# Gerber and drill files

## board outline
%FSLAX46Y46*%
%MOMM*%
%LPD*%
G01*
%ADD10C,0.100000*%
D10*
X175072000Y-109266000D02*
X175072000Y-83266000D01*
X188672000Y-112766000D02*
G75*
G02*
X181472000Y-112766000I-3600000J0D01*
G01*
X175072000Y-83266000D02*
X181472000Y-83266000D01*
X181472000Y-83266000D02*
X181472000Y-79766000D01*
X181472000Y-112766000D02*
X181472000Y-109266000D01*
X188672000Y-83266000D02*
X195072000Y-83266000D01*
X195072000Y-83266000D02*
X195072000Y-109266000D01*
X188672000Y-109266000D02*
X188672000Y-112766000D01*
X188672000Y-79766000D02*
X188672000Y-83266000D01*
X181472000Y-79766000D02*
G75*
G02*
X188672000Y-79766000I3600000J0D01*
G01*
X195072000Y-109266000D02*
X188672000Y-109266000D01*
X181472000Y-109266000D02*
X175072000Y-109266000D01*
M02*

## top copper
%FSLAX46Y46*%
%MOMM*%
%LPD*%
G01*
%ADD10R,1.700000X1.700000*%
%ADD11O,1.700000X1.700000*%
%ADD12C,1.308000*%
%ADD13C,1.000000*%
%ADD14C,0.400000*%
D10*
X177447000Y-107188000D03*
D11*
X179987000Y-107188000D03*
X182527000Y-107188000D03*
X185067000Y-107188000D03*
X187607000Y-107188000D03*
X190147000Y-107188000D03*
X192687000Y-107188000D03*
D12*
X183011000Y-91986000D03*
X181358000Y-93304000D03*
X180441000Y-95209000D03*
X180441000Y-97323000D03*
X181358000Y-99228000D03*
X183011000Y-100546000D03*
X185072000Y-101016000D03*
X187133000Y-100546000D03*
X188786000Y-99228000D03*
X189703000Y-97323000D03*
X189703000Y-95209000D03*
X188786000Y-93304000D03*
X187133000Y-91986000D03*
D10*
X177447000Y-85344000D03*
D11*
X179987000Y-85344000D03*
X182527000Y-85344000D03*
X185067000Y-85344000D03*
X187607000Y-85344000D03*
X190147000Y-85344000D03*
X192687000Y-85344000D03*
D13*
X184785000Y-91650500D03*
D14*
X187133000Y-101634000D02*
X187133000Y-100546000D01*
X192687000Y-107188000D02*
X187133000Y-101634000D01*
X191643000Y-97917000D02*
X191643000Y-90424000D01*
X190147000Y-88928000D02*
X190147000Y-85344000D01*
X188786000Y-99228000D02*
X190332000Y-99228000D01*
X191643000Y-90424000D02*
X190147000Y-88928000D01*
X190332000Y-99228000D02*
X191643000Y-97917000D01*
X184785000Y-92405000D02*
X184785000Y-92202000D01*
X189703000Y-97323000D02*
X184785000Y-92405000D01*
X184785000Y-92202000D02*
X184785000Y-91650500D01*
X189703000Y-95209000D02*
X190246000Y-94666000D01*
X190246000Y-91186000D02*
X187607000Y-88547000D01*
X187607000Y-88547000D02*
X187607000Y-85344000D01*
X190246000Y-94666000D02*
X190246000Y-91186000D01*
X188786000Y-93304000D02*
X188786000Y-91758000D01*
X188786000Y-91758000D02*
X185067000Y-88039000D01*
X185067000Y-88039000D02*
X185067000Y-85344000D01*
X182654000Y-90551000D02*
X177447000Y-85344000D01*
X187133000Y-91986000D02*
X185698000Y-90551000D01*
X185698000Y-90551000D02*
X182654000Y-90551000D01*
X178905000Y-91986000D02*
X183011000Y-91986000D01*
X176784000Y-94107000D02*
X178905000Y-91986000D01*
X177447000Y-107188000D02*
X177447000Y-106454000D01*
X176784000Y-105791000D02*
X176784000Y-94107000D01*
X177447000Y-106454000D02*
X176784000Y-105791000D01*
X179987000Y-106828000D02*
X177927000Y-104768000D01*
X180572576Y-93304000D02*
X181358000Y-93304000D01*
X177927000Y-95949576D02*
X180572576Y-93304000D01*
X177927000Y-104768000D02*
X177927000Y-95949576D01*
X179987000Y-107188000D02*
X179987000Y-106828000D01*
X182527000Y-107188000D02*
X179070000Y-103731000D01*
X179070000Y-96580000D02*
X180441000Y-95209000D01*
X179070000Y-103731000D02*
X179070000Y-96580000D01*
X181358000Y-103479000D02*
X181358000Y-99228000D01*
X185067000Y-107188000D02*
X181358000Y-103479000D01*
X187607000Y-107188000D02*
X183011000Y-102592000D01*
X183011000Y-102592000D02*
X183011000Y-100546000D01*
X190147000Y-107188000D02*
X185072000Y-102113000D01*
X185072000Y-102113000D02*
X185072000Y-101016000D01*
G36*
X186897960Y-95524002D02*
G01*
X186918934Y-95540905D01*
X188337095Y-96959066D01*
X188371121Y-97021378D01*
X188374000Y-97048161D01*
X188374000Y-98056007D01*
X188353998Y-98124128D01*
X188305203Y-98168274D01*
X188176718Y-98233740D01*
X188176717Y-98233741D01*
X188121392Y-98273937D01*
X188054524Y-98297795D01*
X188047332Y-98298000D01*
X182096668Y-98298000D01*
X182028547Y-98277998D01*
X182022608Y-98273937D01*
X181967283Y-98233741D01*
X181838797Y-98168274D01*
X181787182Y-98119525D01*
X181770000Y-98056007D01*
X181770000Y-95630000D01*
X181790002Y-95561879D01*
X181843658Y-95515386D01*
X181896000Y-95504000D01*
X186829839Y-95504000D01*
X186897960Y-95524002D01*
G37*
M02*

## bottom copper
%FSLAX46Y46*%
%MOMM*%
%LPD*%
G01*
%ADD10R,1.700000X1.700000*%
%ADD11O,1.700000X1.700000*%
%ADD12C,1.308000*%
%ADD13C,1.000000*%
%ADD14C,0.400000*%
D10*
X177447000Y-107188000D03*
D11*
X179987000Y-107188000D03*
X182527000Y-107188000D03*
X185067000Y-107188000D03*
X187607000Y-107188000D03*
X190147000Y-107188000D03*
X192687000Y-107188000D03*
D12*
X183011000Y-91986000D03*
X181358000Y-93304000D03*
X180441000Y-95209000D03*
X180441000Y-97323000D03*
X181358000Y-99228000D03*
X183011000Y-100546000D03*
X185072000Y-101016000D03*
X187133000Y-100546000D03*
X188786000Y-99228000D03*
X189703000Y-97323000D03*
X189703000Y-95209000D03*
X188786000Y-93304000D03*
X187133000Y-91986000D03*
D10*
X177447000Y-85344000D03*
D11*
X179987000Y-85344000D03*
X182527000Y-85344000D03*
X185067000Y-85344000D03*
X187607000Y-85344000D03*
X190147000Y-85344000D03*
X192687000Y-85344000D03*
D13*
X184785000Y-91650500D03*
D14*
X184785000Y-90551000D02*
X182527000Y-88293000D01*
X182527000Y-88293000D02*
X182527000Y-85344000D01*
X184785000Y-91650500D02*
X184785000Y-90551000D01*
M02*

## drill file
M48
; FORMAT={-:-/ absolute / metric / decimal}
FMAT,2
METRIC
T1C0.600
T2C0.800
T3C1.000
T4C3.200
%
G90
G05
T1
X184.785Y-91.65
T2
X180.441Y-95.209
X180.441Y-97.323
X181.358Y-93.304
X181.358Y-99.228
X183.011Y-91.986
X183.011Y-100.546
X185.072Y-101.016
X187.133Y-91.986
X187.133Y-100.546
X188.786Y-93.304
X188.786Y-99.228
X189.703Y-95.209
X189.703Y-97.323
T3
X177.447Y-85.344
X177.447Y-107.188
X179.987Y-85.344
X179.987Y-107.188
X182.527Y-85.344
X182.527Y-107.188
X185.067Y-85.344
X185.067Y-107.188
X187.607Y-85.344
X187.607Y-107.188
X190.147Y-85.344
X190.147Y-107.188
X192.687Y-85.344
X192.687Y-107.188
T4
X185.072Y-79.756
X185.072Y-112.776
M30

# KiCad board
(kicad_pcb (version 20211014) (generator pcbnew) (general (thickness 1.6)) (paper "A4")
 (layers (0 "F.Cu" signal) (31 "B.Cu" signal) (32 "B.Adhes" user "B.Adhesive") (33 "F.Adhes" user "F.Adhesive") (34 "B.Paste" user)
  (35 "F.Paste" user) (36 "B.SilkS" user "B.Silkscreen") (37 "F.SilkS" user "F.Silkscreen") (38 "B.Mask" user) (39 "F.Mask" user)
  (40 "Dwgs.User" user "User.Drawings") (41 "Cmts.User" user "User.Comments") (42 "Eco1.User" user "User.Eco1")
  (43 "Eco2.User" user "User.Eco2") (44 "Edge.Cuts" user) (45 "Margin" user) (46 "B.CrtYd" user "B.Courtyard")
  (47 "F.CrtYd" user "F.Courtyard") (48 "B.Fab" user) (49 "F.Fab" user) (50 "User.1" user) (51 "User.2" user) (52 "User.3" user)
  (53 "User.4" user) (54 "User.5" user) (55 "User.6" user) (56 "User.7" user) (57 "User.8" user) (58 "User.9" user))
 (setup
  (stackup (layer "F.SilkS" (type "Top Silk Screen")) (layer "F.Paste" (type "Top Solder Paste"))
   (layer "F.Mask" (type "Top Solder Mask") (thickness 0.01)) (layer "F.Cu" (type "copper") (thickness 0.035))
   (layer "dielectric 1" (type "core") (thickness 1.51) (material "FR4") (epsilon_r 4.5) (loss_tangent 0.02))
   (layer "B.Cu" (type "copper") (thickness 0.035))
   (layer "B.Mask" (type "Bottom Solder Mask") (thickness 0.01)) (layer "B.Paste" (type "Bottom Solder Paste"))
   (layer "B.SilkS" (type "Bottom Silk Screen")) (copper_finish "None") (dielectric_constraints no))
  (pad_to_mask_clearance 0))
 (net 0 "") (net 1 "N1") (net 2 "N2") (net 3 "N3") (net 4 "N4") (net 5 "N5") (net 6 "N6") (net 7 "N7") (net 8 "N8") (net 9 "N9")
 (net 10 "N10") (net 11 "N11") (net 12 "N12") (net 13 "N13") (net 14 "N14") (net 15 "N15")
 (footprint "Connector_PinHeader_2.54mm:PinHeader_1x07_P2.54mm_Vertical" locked (layer "F.Cu") (at 177.447 107.188 90)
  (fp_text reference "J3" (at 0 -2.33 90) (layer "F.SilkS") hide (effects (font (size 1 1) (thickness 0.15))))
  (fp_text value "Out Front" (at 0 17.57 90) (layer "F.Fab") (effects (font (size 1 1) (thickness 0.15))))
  (pad "1" thru_hole rect locked (at 0 0 90) (size 1.7 1.7) (drill 1) (layers *.Cu *.Mask) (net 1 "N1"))
  (pad "2" thru_hole oval locked (at 0 2.54 90) (size 1.7 1.7) (drill 1) (layers *.Cu *.Mask) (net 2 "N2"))
  (pad "3" thru_hole oval locked (at 0 5.08 90) (size 1.7 1.7) (drill 1) (layers *.Cu *.Mask) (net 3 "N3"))
  (pad "4" thru_hole oval locked (at 0 7.62 90) (size 1.7 1.7) (drill 1) (layers *.Cu *.Mask) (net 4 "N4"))
  (pad "5" thru_hole oval locked (at 0 10.16 90) (size 1.7 1.7) (drill 1) (layers *.Cu *.Mask) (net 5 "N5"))
  (pad "6" thru_hole oval locked (at 0 12.7 90) (size 1.7 1.7) (drill 1) (layers *.Cu *.Mask) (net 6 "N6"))
  (pad "7" thru_hole oval locked (at 0 15.24 90) (size 1.7 1.7) (drill 1) (layers *.Cu *.Mask) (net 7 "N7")))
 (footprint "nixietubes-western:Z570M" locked (layer "F.Cu") (at 185.072 96.266 180)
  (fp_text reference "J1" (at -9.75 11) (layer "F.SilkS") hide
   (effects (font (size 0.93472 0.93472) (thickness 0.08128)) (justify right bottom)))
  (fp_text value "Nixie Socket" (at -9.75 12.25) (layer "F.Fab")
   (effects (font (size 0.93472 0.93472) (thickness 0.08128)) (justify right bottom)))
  (pad "1" thru_hole circle locked (at 2.061 4.28 180) (size 1.308 1.308) (drill 0.8) (layers *.Cu *.Mask) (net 1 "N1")
   (solder_mask_margin 0.1016))
  (pad "2" thru_hole circle locked (at 3.714 2.962 180) (size 1.308 1.308) (drill 0.8) (layers *.Cu *.Mask) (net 2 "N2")
   (solder_mask_margin 0.1016))
  (pad "3" thru_hole circle locked (at 4.631 1.057 180) (size 1.308 1.308) (drill 0.8) (layers *.Cu *.Mask) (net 3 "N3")
   (solder_mask_margin 0.1016))
  (pad "4" thru_hole circle locked (at 4.631 -1.057 180) (size 1.308 1.308) (drill 0.8) (layers *.Cu *.Mask) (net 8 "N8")
   (solder_mask_margin 0.1016))
  (pad "5" thru_hole circle locked (at 3.714 -2.962 180) (size 1.308 1.308) (drill 0.8) (layers *.Cu *.Mask) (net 4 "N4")
   (solder_mask_margin 0.1016))
  (pad "6" thru_hole circle locked (at 2.061 -4.28 180) (size 1.308 1.308) (drill 0.8) (layers *.Cu *.Mask) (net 5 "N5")
   (solder_mask_margin 0.1016))
  (pad "7" thru_hole circle locked (at 0 -4.75 180) (size 1.308 1.308) (drill 0.8) (layers *.Cu *.Mask) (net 6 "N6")
   (solder_mask_margin 0.1016))
  (pad "8" thru_hole circle locked (at -2.061 -4.28 180) (size 1.308 1.308) (drill 0.8) (layers *.Cu *.Mask) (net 7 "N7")
   (solder_mask_margin 0.1016))
  (pad "9" thru_hole circle locked (at -3.714 -2.962 180) (size 1.308 1.308) (drill 0.8) (layers *.Cu *.Mask) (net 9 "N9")
   (solder_mask_margin 0.1016))
  (pad "10" thru_hole circle locked (at -4.631 -1.057 180) (size 1.308 1.308) (drill 0.8) (layers *.Cu *.Mask) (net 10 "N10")
   (solder_mask_margin 0.1016))
  (pad "11" thru_hole circle locked (at -4.631 1.057 180) (size 1.308 1.308) (drill 0.8) (layers *.Cu *.Mask) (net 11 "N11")
   (solder_mask_margin 0.1016))
  (pad "12" thru_hole circle locked (at -3.714 2.962 180) (size 1.308 1.308) (drill 0.8) (layers *.Cu *.Mask) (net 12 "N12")
   (solder_mask_margin 0.1016))
  (pad "13" thru_hole circle locked (at -2.061 4.28 180) (size 1.308 1.308) (drill 0.8) (layers *.Cu *.Mask) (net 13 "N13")
   (solder_mask_margin 0.1016)))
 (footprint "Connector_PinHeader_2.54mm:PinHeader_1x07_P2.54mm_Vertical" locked (layer "F.Cu") (at 177.447 85.344 90)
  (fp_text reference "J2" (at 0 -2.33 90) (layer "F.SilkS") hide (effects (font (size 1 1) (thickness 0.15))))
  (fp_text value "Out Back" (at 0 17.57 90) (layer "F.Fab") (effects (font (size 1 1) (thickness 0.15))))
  (pad "1" thru_hole rect locked (at 0 0 90) (size 1.7 1.7) (drill 1) (layers *.Cu *.Mask) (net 13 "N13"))
  (pad "2" thru_hole oval locked (at 0 2.54 90) (size 1.7 1.7) (drill 1) (layers *.Cu *.Mask) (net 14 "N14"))
  (pad "3" thru_hole oval locked (at 0 5.08 90) (size 1.7 1.7) (drill 1) (layers *.Cu *.Mask) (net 10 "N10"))
  (pad "4" thru_hole oval locked (at 0 7.62 90) (size 1.7 1.7) (drill 1) (layers *.Cu *.Mask) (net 12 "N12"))
  (pad "5" thru_hole oval locked (at 0 10.16 90) (size 1.7 1.7) (drill 1) (layers *.Cu *.Mask) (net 11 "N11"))
  (pad "6" thru_hole oval locked (at 0 12.7 90) (size 1.7 1.7) (drill 1) (layers *.Cu *.Mask) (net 9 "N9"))
  (pad "7" thru_hole oval locked (at 0 15.24 90) (size 1.7 1.7) (drill 1) (layers *.Cu *.Mask) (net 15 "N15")))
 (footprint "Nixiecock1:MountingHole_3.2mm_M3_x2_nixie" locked (layer "F.Cu") (at 185.072 96.266 90)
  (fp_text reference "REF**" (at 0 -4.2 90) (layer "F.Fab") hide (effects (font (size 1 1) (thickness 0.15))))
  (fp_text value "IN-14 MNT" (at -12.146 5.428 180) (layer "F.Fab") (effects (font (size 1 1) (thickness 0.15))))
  (pad "" np_thru_hole circle locked (at -16.51 0 90) (size 3.2 3.2) (drill 3.2) (layers F&B.Cu *.Mask))
  (pad "" np_thru_hole circle locked (at 16.51 0 90) (size 3.2 3.2) (drill 3.2) (layers F&B.Cu *.Mask)))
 (gr_line locked (start 175.072 109.266) (end 175.072 83.266) (layer "Edge.Cuts") (width 0.1))
 (gr_arc locked (start 188.672 112.766) (mid 185.072 116.366) (end 181.472 112.766) (layer "Edge.Cuts") (width 0.1))
 (gr_line locked (start 175.072 83.266) (end 181.472 83.266) (layer "Edge.Cuts") (width 0.1))
 (gr_line locked (start 181.472 83.266) (end 181.472 79.766) (layer "Edge.Cuts") (width 0.1))
 (gr_line locked (start 181.472 112.766) (end 181.472 109.266) (layer "Edge.Cuts") (width 0.1))
 (gr_line locked (start 188.672 83.266) (end 195.072 83.266) (layer "Edge.Cuts") (width 0.1))
 (gr_line locked (start 195.072 83.266) (end 195.072 109.266) (layer "Edge.Cuts") (width 0.1))
 (gr_line locked (start 188.672 109.266) (end 188.672 112.766) (layer "Edge.Cuts") (width 0.1))
 (gr_line locked (start 188.672 79.766) (end 188.672 83.266) (layer "Edge.Cuts") (width 0.1))
 (gr_arc locked (start 181.472 79.766) (mid 185.072 76.166) (end 188.672 79.766) (layer "Edge.Cuts") (width 0.1))
 (gr_line locked (start 195.072 109.266) (end 188.672 109.266) (layer "Edge.Cuts") (width 0.1))
 (gr_line locked (start 181.472 109.266) (end 175.072 109.266) (layer "Edge.Cuts") (width 0.1))
 (segment (start 187.133 101.634) (end 187.133 100.546) (width 0.4) (layer "F.Cu") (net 7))
 (segment (start 192.687 107.188) (end 187.133 101.634) (width 0.4) (layer "F.Cu") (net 7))
 (segment (start 191.643 97.917) (end 191.643 90.424) (width 0.4) (layer "F.Cu") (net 9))
 (segment (start 190.147 88.928) (end 190.147 85.344) (width 0.4) (layer "F.Cu") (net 9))
 (segment (start 188.786 99.228) (end 190.332 99.228) (width 0.4) (layer "F.Cu") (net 9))
 (segment (start 191.643 90.424) (end 190.147 88.928) (width 0.4) (layer "F.Cu") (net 9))
 (segment (start 190.332 99.228) (end 191.643 97.917) (width 0.4) (layer "F.Cu") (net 9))
 (segment (start 184.785 92.405) (end 184.785 92.202) (width 0.4) (layer "F.Cu") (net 10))
 (segment (start 189.703 97.323) (end 184.785 92.405) (width 0.4) (layer "F.Cu") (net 10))
 (segment (start 184.785 92.202) (end 184.785 91.6505) (width 0.4) (layer "F.Cu") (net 10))
 (via (at 184.785 91.6505) (size 1) (drill 0.6) (layers "F.Cu" "B.Cu") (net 10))
 (segment (start 184.785 90.551) (end 182.527 88.293) (width 0.4) (layer "B.Cu") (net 10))
 (segment (start 182.527 88.293) (end 182.527 85.344) (width 0.4) (layer "B.Cu") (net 10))
 (segment (start 184.785 91.6505) (end 184.785 90.551) (width 0.4) (layer "B.Cu") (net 10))
 (segment (start 189.703 95.209) (end 190.246 94.666) (width 0.4) (layer "F.Cu") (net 11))
 (segment (start 190.246 91.186) (end 187.607 88.547) (width 0.4) (layer "F.Cu") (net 11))
 (segment (start 187.607 88.547) (end 187.607 85.344) (width 0.4) (layer "F.Cu") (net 11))
 (segment (start 190.246 94.666) (end 190.246 91.186) (width 0.4) (layer "F.Cu") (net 11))
 (segment (start 188.786 93.304) (end 188.786 91.758) (width 0.4) (layer "F.Cu") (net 12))
 (segment (start 188.786 91.758) (end 185.067 88.039) (width 0.4) (layer "F.Cu") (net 12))
 (segment (start 185.067 88.039) (end 185.067 85.344) (width 0.4) (layer "F.Cu") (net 12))
 (segment (start 182.654 90.551) (end 177.447 85.344) (width 0.4) (layer "F.Cu") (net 13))
 (segment (start 187.133 91.986) (end 185.698 90.551) (width 0.4) (layer "F.Cu") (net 13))
 (segment (start 185.698 90.551) (end 182.654 90.551) (width 0.4) (layer "F.Cu") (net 13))
 (segment (start 178.905 91.986) (end 183.011 91.986) (width 0.4) (layer "F.Cu") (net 1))
 (segment (start 176.784 94.107) (end 178.905 91.986) (width 0.4) (layer "F.Cu") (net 1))
 (segment (start 177.447 107.188) (end 177.447 106.454) (width 0.4) (layer "F.Cu") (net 1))
 (segment (start 176.784 105.791) (end 176.784 94.107) (width 0.4) (layer "F.Cu") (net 1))
 (segment (start 177.447 106.454) (end 176.784 105.791) (width 0.4) (layer "F.Cu") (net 1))
 (segment (start 179.987 106.828) (end 177.927 104.768) (width 0.4) (layer "F.Cu") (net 2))
 (segment (start 180.572576 93.304) (end 181.358 93.304) (width 0.4) (layer "F.Cu") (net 2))
 (segment (start 177.927 95.949576) (end 180.572576 93.304) (width 0.4) (layer "F.Cu") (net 2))
 (segment (start 177.927 104.768) (end 177.927 95.949576) (width 0.4) (layer "F.Cu") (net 2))
 (segment (start 179.987 107.188) (end 179.987 106.828) (width 0.4) (layer "F.Cu") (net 2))
 (segment (start 182.527 107.188) (end 179.07 103.731) (width 0.4) (layer "F.Cu") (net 3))
 (segment (start 179.07 96.58) (end 180.441 95.209) (width 0.4) (layer "F.Cu") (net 3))
 (segment (start 179.07 103.731) (end 179.07 96.58) (width 0.4) (layer "F.Cu") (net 3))
 (segment (start 181.358 103.479) (end 181.358 99.228) (width 0.4) (layer "F.Cu") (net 4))
 (segment (start 185.067 107.188) (end 181.358 103.479) (width 0.4) (layer "F.Cu") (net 4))
 (segment (start 187.607 107.188) (end 183.011 102.592) (width 0.4) (layer "F.Cu") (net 5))
 (segment (start 183.011 102.592) (end 183.011 100.546) (width 0.4) (layer "F.Cu") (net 5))
 (segment (start 190.147 107.188) (end 185.072 102.113) (width 0.4) (layer "F.Cu") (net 6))
 (segment (start 185.072 102.113) (end 185.072 101.016) (width 0.4) (layer "F.Cu") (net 6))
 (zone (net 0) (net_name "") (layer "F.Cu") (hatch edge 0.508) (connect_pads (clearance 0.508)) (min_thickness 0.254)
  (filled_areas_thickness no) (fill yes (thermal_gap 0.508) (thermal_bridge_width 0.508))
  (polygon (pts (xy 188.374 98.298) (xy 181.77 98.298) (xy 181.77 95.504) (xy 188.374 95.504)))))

